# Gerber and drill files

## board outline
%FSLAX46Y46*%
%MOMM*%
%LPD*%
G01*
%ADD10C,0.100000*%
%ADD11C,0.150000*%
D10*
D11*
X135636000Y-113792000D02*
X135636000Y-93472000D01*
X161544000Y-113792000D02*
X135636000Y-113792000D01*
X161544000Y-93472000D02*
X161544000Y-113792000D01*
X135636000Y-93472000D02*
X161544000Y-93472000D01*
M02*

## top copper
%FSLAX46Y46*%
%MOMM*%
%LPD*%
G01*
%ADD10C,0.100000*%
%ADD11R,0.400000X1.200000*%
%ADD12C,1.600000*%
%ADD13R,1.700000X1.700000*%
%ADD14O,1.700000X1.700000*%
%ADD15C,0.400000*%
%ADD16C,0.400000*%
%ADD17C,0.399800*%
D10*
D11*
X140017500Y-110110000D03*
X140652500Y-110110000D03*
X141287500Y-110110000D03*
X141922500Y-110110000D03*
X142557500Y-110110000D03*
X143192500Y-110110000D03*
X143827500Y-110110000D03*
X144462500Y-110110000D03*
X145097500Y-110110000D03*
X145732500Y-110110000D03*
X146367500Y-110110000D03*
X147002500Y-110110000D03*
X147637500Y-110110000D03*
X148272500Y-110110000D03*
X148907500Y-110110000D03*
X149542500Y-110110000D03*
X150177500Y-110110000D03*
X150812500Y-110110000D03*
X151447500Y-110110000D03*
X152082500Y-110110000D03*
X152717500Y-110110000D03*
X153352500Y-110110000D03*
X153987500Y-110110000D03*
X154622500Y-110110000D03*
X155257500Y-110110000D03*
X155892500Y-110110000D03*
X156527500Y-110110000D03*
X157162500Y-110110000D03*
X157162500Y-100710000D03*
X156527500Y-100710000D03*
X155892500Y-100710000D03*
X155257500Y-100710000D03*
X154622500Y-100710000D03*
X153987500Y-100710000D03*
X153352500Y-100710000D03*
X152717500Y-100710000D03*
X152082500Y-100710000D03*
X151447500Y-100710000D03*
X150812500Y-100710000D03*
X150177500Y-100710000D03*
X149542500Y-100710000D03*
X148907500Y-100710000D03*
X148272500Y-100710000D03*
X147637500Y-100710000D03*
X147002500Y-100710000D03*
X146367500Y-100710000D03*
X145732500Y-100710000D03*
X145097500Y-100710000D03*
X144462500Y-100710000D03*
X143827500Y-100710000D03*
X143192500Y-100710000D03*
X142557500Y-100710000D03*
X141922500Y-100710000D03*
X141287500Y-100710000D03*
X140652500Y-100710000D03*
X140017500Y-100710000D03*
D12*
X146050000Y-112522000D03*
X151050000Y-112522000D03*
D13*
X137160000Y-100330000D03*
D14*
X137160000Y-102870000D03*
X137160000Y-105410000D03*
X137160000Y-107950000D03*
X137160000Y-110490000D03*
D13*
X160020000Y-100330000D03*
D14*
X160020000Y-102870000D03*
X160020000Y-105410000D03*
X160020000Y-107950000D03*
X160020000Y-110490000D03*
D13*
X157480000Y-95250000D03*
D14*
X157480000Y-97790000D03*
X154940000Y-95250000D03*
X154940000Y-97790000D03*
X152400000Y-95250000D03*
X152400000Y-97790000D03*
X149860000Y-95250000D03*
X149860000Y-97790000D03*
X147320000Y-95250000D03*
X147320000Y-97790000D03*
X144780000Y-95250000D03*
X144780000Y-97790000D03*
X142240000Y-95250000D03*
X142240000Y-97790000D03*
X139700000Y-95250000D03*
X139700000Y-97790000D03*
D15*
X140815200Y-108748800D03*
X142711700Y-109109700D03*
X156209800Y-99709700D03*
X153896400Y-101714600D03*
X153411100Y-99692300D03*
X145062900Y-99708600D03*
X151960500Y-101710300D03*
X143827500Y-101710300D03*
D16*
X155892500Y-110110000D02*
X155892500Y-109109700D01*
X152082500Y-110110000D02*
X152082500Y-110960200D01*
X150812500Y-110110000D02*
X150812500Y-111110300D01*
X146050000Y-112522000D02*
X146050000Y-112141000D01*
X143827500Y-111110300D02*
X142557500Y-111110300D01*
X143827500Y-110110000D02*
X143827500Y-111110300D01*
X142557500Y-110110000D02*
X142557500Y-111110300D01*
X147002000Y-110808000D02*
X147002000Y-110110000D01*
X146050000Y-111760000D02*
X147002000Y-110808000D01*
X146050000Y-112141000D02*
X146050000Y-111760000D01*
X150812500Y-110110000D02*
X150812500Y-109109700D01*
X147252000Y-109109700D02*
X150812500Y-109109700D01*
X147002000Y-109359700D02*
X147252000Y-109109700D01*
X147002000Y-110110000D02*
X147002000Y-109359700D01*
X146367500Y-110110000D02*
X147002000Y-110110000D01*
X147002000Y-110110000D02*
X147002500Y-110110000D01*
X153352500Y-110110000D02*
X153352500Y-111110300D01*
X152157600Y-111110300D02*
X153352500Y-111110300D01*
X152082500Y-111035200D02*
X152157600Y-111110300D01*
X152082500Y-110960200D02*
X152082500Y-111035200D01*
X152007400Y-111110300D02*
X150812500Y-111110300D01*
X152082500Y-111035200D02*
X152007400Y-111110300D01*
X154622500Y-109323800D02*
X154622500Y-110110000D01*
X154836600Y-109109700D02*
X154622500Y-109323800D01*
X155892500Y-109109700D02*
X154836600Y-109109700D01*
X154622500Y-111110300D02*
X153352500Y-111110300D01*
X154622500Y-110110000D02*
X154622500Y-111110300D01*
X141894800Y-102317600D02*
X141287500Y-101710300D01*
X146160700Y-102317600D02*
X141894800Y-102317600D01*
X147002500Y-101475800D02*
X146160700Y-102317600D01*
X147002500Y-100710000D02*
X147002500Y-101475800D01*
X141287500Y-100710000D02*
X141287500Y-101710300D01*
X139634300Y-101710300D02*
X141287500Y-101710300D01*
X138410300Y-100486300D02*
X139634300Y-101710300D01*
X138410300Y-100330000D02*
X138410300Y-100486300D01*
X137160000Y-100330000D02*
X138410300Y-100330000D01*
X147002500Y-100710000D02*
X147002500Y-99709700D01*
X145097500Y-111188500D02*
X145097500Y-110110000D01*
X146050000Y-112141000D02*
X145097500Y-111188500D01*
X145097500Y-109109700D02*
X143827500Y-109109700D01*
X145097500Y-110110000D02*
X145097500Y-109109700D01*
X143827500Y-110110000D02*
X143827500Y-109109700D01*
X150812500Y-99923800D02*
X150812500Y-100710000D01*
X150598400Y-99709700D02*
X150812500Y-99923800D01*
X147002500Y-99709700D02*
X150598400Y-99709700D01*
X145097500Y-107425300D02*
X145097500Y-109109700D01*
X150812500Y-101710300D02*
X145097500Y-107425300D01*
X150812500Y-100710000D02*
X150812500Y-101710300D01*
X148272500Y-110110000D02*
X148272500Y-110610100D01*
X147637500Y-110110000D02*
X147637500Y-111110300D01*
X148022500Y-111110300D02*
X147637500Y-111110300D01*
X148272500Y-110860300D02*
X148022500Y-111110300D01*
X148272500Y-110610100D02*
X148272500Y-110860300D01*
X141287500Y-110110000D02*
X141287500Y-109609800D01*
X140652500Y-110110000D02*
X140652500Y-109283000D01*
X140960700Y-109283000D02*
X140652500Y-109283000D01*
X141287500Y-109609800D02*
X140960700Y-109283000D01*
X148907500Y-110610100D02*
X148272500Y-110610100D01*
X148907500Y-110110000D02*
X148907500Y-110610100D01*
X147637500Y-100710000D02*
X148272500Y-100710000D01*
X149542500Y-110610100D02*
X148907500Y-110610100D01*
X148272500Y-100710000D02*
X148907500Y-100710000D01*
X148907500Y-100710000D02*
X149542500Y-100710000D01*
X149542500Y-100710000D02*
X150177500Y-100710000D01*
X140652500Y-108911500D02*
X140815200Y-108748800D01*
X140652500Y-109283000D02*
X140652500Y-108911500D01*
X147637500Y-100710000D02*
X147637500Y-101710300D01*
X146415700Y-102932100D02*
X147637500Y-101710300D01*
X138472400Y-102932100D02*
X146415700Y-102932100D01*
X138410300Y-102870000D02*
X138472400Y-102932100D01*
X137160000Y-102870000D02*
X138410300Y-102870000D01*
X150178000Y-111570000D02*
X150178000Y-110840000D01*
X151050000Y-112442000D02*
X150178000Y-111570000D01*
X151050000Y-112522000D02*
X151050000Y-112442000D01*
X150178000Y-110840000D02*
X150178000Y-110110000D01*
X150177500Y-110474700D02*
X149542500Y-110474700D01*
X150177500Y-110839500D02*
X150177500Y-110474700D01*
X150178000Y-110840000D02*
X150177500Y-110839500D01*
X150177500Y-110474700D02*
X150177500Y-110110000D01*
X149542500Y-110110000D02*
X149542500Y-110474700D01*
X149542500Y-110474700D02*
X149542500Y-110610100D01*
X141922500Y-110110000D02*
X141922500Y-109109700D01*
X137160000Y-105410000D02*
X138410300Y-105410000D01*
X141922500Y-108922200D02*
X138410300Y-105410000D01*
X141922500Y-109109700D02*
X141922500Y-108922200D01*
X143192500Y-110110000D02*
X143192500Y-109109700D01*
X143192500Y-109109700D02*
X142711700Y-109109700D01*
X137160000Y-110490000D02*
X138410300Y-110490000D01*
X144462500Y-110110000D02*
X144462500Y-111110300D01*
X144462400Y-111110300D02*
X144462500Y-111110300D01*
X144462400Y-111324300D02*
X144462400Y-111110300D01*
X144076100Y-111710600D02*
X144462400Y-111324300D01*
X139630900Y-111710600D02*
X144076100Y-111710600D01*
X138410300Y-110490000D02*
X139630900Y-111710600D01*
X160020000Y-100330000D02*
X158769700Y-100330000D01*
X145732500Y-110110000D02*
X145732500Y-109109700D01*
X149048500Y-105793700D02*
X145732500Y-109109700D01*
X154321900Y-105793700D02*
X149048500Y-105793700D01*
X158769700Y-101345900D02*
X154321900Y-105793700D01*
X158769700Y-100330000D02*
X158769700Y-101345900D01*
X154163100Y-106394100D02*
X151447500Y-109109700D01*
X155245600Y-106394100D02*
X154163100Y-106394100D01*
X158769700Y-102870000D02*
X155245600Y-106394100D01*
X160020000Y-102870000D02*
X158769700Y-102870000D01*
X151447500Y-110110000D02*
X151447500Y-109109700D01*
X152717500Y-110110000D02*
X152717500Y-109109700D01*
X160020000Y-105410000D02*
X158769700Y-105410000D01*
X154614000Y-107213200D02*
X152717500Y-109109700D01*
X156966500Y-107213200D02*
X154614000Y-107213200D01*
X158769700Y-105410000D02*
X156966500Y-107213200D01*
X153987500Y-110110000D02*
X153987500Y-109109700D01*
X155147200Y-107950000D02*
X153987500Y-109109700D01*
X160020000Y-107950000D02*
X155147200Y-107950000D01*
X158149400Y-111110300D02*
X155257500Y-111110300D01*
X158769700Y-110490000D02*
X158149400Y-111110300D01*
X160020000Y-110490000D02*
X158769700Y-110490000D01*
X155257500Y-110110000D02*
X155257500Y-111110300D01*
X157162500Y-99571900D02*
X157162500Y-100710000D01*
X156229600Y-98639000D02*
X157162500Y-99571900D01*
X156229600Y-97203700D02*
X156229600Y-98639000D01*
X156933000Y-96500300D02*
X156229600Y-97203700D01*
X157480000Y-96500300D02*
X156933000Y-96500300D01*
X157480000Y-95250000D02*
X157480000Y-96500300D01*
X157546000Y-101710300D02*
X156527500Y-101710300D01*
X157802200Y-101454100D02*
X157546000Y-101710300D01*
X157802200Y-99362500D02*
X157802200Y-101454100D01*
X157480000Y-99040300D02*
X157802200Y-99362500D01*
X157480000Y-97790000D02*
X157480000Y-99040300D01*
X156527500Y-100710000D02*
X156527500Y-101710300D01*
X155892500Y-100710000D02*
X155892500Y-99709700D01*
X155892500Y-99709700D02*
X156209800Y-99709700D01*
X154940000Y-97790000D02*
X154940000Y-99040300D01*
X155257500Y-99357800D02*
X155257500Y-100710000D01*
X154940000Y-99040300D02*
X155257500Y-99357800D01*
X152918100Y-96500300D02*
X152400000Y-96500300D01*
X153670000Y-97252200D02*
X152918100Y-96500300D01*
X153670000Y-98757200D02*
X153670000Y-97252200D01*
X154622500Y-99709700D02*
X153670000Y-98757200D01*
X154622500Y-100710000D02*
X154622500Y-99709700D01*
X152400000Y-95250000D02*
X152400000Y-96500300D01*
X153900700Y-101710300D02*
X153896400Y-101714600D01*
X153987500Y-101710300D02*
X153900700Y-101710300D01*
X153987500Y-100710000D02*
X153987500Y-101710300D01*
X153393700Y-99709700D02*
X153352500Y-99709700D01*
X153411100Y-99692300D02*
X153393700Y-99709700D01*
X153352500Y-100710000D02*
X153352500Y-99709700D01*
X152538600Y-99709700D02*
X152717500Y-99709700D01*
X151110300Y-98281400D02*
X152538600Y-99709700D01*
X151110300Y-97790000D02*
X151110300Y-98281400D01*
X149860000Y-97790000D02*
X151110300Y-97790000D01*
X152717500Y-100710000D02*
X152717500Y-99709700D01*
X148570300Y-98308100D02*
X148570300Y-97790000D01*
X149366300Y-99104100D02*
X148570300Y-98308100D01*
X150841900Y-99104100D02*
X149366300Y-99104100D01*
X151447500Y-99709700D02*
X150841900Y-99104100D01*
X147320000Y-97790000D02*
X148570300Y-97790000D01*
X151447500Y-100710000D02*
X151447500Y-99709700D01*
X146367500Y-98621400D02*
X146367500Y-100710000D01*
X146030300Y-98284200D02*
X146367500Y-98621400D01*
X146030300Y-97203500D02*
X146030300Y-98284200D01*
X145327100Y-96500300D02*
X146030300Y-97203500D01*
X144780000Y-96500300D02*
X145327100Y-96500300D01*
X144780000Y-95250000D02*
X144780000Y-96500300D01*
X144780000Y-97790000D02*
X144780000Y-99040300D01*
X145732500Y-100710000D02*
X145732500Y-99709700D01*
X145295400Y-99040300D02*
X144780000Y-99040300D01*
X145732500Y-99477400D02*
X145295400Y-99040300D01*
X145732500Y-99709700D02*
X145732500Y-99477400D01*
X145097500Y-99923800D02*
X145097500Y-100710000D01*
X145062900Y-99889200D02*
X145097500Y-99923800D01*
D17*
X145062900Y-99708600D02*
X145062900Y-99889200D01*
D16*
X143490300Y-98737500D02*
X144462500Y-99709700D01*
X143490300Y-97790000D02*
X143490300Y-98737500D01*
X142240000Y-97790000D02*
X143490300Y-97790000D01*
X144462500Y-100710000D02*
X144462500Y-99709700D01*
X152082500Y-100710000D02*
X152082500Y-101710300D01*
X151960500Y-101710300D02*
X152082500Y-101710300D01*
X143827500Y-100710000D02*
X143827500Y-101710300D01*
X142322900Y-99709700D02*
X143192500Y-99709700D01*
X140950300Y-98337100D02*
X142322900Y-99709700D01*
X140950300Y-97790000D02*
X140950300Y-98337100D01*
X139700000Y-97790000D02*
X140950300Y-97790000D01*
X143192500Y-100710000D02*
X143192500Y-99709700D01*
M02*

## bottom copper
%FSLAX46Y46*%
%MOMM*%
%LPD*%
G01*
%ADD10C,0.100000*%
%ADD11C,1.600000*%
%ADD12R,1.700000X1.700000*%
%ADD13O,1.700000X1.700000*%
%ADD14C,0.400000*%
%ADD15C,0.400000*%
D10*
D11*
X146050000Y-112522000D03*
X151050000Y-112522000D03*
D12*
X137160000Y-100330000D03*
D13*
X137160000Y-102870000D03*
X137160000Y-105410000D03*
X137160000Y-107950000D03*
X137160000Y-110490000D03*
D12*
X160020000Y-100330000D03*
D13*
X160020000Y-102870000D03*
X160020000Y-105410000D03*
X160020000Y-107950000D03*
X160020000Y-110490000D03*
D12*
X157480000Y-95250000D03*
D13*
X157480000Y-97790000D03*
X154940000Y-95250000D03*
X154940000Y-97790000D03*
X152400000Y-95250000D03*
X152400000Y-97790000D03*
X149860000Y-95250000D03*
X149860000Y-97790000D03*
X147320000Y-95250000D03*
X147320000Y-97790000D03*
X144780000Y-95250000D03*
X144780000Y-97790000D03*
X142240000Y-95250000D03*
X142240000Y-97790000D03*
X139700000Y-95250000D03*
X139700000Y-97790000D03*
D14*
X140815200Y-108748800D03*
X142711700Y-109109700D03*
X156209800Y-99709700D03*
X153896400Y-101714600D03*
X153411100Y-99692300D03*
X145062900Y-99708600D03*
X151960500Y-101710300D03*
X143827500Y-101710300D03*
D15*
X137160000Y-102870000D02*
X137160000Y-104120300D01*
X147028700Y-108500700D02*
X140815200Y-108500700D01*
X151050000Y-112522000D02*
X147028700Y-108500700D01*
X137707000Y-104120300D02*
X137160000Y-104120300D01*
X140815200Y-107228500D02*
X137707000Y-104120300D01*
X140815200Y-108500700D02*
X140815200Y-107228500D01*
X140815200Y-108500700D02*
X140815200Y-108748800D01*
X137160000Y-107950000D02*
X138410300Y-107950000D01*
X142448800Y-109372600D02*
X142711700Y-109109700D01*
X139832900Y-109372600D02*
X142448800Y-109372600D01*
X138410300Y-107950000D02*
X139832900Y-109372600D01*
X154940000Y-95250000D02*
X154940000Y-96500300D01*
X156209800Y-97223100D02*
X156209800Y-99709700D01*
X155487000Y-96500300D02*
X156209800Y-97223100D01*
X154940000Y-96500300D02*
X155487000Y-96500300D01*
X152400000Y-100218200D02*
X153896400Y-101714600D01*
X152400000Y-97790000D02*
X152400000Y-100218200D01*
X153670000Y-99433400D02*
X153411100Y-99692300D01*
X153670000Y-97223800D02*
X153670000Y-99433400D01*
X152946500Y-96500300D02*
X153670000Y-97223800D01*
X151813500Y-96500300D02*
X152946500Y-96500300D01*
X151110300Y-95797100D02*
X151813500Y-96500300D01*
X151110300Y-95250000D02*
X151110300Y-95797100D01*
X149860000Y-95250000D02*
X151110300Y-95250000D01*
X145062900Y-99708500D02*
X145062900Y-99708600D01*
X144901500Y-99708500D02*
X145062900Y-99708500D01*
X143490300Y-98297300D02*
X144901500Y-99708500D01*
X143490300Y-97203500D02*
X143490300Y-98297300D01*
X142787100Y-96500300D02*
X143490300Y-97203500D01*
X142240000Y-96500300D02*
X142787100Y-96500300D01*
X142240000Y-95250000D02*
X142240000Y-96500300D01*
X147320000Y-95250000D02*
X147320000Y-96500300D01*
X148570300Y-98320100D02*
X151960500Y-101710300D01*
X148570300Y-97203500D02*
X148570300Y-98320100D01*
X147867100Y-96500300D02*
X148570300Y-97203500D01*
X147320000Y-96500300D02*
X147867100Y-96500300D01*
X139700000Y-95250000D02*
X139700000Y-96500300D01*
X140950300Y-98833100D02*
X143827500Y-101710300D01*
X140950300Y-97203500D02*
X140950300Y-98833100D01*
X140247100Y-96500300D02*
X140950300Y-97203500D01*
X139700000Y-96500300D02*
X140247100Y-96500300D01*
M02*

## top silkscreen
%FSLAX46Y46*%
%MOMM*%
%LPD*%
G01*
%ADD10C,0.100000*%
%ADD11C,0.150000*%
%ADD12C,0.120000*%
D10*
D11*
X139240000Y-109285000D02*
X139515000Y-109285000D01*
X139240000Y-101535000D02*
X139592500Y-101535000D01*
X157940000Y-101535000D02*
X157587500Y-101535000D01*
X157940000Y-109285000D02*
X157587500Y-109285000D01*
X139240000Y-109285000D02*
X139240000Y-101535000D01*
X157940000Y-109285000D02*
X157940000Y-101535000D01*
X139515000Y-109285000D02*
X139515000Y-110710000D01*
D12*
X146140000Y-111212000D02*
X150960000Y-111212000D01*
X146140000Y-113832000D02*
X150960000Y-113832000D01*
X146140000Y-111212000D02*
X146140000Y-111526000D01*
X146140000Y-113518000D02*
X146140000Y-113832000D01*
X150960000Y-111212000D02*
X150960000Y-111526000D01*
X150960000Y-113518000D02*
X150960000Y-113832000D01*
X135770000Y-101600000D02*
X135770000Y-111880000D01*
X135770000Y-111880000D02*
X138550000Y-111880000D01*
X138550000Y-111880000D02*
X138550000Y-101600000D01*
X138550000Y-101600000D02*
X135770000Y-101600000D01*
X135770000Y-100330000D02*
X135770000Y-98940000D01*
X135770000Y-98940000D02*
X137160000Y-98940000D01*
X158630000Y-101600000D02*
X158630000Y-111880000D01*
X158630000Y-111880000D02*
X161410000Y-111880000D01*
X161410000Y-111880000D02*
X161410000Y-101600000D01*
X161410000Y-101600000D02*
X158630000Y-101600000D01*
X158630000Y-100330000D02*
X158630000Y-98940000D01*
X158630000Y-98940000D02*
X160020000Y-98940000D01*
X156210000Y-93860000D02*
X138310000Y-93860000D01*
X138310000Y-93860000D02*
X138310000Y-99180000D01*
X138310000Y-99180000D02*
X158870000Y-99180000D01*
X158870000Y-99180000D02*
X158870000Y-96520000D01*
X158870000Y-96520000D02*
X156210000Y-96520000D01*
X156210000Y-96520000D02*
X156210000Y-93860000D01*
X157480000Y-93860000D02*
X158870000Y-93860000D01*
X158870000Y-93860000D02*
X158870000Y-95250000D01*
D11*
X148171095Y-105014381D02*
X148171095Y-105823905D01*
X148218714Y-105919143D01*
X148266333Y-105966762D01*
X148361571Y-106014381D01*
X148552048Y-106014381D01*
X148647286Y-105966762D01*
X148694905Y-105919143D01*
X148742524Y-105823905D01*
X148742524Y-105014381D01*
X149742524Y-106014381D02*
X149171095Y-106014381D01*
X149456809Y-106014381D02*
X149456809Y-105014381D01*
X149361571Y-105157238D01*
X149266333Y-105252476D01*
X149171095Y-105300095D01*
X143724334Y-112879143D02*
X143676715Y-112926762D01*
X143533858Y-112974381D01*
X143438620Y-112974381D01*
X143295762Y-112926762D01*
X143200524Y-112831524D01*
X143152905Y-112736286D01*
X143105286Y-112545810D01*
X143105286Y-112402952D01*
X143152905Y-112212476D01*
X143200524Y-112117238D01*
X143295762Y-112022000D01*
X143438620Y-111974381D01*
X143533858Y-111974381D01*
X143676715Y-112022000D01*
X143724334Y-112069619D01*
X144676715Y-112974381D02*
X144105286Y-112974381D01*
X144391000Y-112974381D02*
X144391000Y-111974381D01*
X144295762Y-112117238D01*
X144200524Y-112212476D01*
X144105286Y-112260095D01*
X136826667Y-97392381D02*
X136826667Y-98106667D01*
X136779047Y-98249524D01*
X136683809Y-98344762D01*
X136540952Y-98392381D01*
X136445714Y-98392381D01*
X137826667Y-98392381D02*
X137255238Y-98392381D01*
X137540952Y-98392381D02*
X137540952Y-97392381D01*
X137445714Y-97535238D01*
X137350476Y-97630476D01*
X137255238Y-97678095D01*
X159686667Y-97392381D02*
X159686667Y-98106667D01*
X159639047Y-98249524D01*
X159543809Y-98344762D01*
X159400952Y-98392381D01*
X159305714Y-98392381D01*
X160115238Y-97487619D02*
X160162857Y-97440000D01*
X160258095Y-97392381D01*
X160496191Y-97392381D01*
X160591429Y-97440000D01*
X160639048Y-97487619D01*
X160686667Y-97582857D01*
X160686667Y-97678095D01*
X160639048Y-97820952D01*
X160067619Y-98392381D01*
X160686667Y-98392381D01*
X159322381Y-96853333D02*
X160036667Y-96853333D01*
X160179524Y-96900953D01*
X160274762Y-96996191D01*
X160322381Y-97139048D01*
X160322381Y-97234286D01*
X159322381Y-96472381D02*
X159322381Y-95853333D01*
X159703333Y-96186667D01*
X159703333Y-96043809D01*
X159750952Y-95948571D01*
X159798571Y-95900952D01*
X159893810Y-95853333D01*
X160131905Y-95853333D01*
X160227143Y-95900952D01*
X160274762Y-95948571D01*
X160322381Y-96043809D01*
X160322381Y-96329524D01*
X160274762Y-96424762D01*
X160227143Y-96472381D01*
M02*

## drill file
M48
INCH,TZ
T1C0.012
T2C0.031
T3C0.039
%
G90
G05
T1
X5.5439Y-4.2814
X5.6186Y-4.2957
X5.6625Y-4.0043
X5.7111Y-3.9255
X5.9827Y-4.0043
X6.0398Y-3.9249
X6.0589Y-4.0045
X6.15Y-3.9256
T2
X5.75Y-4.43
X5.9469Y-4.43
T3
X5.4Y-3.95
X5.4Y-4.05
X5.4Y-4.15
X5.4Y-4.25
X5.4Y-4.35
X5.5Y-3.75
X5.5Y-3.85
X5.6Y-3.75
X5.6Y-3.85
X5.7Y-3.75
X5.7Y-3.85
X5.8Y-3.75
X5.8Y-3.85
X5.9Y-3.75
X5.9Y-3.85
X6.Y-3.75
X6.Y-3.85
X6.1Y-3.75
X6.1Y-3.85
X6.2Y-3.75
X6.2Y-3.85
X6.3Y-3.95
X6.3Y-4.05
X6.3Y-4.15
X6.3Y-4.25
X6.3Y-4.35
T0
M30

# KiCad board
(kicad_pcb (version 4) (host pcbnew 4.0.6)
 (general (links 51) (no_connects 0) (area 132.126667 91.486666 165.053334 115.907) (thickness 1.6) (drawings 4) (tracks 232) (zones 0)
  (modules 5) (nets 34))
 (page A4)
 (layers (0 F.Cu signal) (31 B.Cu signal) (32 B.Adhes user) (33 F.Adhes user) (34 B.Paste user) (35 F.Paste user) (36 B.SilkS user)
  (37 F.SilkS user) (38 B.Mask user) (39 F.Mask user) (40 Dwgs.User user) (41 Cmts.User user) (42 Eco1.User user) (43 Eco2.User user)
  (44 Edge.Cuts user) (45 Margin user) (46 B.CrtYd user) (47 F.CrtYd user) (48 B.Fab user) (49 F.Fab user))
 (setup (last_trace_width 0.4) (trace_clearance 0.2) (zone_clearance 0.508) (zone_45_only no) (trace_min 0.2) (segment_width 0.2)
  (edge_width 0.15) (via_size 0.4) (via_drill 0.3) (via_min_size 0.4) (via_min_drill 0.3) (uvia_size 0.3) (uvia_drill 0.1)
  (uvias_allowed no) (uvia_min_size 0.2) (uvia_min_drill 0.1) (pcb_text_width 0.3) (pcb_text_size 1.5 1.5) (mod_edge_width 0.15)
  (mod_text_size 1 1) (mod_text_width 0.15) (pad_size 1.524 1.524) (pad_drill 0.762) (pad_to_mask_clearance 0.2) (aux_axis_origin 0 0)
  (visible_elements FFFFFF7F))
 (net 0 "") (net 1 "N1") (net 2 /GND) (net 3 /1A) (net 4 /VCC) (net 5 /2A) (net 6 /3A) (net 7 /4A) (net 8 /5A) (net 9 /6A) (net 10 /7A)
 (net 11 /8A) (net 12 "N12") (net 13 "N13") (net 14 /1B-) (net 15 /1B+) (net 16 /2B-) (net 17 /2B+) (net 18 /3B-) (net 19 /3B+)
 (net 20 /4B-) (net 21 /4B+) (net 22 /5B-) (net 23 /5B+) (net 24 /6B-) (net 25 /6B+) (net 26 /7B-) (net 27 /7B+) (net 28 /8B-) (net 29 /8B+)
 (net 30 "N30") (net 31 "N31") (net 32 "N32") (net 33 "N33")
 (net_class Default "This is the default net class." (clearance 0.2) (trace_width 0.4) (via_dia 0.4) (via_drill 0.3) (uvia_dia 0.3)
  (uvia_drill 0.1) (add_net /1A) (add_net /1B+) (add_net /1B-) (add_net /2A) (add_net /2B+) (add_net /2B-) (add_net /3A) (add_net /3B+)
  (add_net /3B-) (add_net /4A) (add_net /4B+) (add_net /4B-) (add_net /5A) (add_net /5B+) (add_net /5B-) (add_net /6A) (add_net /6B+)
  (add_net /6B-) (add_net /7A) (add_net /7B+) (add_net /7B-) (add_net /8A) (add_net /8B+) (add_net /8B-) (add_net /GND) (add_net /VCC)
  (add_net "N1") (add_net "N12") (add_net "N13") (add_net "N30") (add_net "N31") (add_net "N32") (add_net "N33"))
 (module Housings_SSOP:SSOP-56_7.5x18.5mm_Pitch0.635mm (layer F.Cu) (at 148.59 105.41 90)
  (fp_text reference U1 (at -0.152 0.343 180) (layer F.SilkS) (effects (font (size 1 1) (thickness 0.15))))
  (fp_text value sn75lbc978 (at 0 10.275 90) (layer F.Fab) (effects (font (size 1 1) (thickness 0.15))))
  (fp_line (start -3.875 -9.35) (end -3.875 -9.075) (layer F.SilkS) (width 0.15))
  (fp_line (start 3.875 -9.35) (end 3.875 -8.9975) (layer F.SilkS) (width 0.15))
  (fp_line (start 3.875 9.35) (end 3.875 8.9975) (layer F.SilkS) (width 0.15))
  (fp_line (start -3.875 9.35) (end -3.875 8.9975) (layer F.SilkS) (width 0.15))
  (fp_line (start -3.875 -9.35) (end 3.875 -9.35) (layer F.SilkS) (width 0.15))
  (fp_line (start -3.875 9.35) (end 3.875 9.35) (layer F.SilkS) (width 0.15))
  (fp_line (start -3.875 -9.075) (end -5.3 -9.075) (layer F.SilkS) (width 0.15))
  (pad 1 smd rect (at -4.7 -8.5725 90) (size 1.2 0.4) (layers F.Cu F.Paste F.Mask) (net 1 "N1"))
  (pad 2 smd rect (at -4.7 -7.9375 90) (size 1.2 0.4) (layers F.Cu F.Paste F.Mask) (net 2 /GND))
  (pad 3 smd rect (at -4.7 -7.3025 90) (size 1.2 0.4) (layers F.Cu F.Paste F.Mask) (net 2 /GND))
  (pad 4 smd rect (at -4.7 -6.6675 90) (size 1.2 0.4) (layers F.Cu F.Paste F.Mask) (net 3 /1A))
  (pad 5 smd rect (at -4.7 -6.0325 90) (size 1.2 0.4) (layers F.Cu F.Paste F.Mask) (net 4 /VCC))
  (pad 6 smd rect (at -4.7 -5.3975 90) (size 1.2 0.4) (layers F.Cu F.Paste F.Mask) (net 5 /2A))
  (pad 7 smd rect (at -4.7 -4.7625 90) (size 1.2 0.4) (layers F.Cu F.Paste F.Mask) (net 4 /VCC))
  (pad 8 smd rect (at -4.7 -4.1275 90) (size 1.2 0.4) (layers F.Cu F.Paste F.Mask) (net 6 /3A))
  (pad 9 smd rect (at -4.7 -3.4925 90) (size 1.2 0.4) (layers F.Cu F.Paste F.Mask) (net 4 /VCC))
  (pad 10 smd rect (at -4.7 -2.8575 90) (size 1.2 0.4) (layers F.Cu F.Paste F.Mask) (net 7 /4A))
  (pad 11 smd rect (at -4.7 -2.2225 90) (size 1.2 0.4) (layers F.Cu F.Paste F.Mask) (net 4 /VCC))
  (pad 12 smd rect (at -4.7 -1.5875 90) (size 1.2 0.4) (layers F.Cu F.Paste F.Mask) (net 4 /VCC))
  (pad 13 smd rect (at -4.7 -0.9525 90) (size 1.2 0.4) (layers F.Cu F.Paste F.Mask) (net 2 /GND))
  (pad 14 smd rect (at -4.7 -0.3175 90) (size 1.2 0.4) (layers F.Cu F.Paste F.Mask) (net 2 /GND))
  (pad 15 smd rect (at -4.7 0.3175 90) (size 1.2 0.4) (layers F.Cu F.Paste F.Mask) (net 2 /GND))
  (pad 16 smd rect (at -4.7 0.9525 90) (size 1.2 0.4) (layers F.Cu F.Paste F.Mask) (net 2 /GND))
  (pad 17 smd rect (at -4.7 1.5875 90) (size 1.2 0.4) (layers F.Cu F.Paste F.Mask) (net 2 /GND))
  (pad 18 smd rect (at -4.7 2.2225 90) (size 1.2 0.4) (layers F.Cu F.Paste F.Mask) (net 4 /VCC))
  (pad 19 smd rect (at -4.7 2.8575 90) (size 1.2 0.4) (layers F.Cu F.Paste F.Mask) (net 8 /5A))
  (pad 20 smd rect (at -4.7 3.4925 90) (size 1.2 0.4) (layers F.Cu F.Paste F.Mask) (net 4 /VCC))
  (pad 21 smd rect (at -4.7 4.1275 90) (size 1.2 0.4) (layers F.Cu F.Paste F.Mask) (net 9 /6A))
  (pad 22 smd rect (at -4.7 4.7625 90) (size 1.2 0.4) (layers F.Cu F.Paste F.Mask) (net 4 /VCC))
  (pad 23 smd rect (at -4.7 5.3975 90) (size 1.2 0.4) (layers F.Cu F.Paste F.Mask) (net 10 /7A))
  (pad 24 smd rect (at -4.7 6.0325 90) (size 1.2 0.4) (layers F.Cu F.Paste F.Mask) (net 4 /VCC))
  (pad 25 smd rect (at -4.7 6.6675 90) (size 1.2 0.4) (layers F.Cu F.Paste F.Mask) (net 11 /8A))
  (pad 26 smd rect (at -4.7 7.3025 90) (size 1.2 0.4) (layers F.Cu F.Paste F.Mask) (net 4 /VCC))
  (pad 27 smd rect (at -4.7 7.9375 90) (size 1.2 0.4) (layers F.Cu F.Paste F.Mask) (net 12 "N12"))
  (pad 28 smd rect (at -4.7 8.5725 90) (size 1.2 0.4) (layers F.Cu F.Paste F.Mask) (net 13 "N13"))
  (pad 29 smd rect (at 4.7 8.5725 90) (size 1.2 0.4) (layers F.Cu F.Paste F.Mask) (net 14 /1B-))
  (pad 30 smd rect (at 4.7 7.9375 90) (size 1.2 0.4) (layers F.Cu F.Paste F.Mask) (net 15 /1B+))
  (pad 31 smd rect (at 4.7 7.3025 90) (size 1.2 0.4) (layers F.Cu F.Paste F.Mask) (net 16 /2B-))
  (pad 32 smd rect (at 4.7 6.6675 90) (size 1.2 0.4) (layers F.Cu F.Paste F.Mask) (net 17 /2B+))
  (pad 33 smd rect (at 4.7 6.0325 90) (size 1.2 0.4) (layers F.Cu F.Paste F.Mask) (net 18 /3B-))
  (pad 34 smd rect (at 4.7 5.3975 90) (size 1.2 0.4) (layers F.Cu F.Paste F.Mask) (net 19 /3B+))
  (pad 35 smd rect (at 4.7 4.7625 90) (size 1.2 0.4) (layers F.Cu F.Paste F.Mask) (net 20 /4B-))
  (pad 36 smd rect (at 4.7 4.1275 90) (size 1.2 0.4) (layers F.Cu F.Paste F.Mask) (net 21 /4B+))
  (pad 37 smd rect (at 4.7 3.4925 90) (size 1.2 0.4) (layers F.Cu F.Paste F.Mask) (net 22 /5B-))
  (pad 38 smd rect (at 4.7 2.8575 90) (size 1.2 0.4) (layers F.Cu F.Paste F.Mask) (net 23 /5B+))
  (pad 39 smd rect (at 4.7 2.2225 90) (size 1.2 0.4) (layers F.Cu F.Paste F.Mask) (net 4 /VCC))
  (pad 40 smd rect (at 4.7 1.5875 90) (size 1.2 0.4) (layers F.Cu F.Paste F.Mask) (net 2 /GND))
  (pad 41 smd rect (at 4.7 0.9525 90) (size 1.2 0.4) (layers F.Cu F.Paste F.Mask) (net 2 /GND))
  (pad 42 smd rect (at 4.7 0.3175 90) (size 1.2 0.4) (layers F.Cu F.Paste F.Mask) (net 2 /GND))
  (pad 43 smd rect (at 4.7 -0.3175 90) (size 1.2 0.4) (layers F.Cu F.Paste F.Mask) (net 2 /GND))
  (pad 44 smd rect (at 4.7 -0.9525 90) (size 1.2 0.4) (layers F.Cu F.Paste F.Mask) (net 2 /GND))
  (pad 45 smd rect (at 4.7 -1.5875 90) (size 1.2 0.4) (layers F.Cu F.Paste F.Mask) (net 4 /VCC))
  (pad 46 smd rect (at 4.7 -2.2225 90) (size 1.2 0.4) (layers F.Cu F.Paste F.Mask) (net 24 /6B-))
  (pad 47 smd rect (at 4.7 -2.8575 90) (size 1.2 0.4) (layers F.Cu F.Paste F.Mask) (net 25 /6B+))
  (pad 48 smd rect (at 4.7 -3.4925 90) (size 1.2 0.4) (layers F.Cu F.Paste F.Mask) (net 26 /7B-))
  (pad 49 smd rect (at 4.7 -4.1275 90) (size 1.2 0.4) (layers F.Cu F.Paste F.Mask) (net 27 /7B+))
  (pad 50 smd rect (at 4.7 -4.7625 90) (size 1.2 0.4) (layers F.Cu F.Paste F.Mask) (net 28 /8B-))
  (pad 51 smd rect (at 4.7 -5.3975 90) (size 1.2 0.4) (layers F.Cu F.Paste F.Mask) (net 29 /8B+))
  (pad 52 smd rect (at 4.7 -6.0325 90) (size 1.2 0.4) (layers F.Cu F.Paste F.Mask) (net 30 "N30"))
  (pad 53 smd rect (at 4.7 -6.6675 90) (size 1.2 0.4) (layers F.Cu F.Paste F.Mask) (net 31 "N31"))
  (pad 54 smd rect (at 4.7 -7.3025 90) (size 1.2 0.4) (layers F.Cu F.Paste F.Mask) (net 4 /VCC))
  (pad 55 smd rect (at 4.7 -7.9375 90) (size 1.2 0.4) (layers F.Cu F.Paste F.Mask) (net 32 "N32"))
  (pad 56 smd rect (at 4.7 -8.5725 90) (size 1.2 0.4) (layers F.Cu F.Paste F.Mask) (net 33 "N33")))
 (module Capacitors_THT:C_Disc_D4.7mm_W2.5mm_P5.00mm (layer F.Cu) (at 146.05 112.522)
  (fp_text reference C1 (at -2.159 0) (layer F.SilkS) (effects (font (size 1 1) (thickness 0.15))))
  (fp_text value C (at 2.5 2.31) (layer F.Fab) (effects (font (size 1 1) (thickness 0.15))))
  (fp_line (start 0.09 -1.31) (end 4.91 -1.31) (layer F.SilkS) (width 0.12))
  (fp_line (start 0.09 1.31) (end 4.91 1.31) (layer F.SilkS) (width 0.12))
  (fp_line (start 0.09 -1.31) (end 0.09 -0.996) (layer F.SilkS) (width 0.12))
  (fp_line (start 0.09 0.996) (end 0.09 1.31) (layer F.SilkS) (width 0.12))
  (fp_line (start 4.91 -1.31) (end 4.91 -0.996) (layer F.SilkS) (width 0.12))
  (fp_line (start 4.91 0.996) (end 4.91 1.31) (layer F.SilkS) (width 0.12))
  (pad 1 thru_hole circle (at 0 0) (size 1.6 1.6) (drill 0.8) (layers *.Cu *.Mask) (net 4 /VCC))
  (pad 2 thru_hole circle (at 5 0) (size 1.6 1.6) (drill 0.8) (layers *.Cu *.Mask) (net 2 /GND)))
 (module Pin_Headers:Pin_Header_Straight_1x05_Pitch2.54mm (layer F.Cu) (at 137.16 100.33)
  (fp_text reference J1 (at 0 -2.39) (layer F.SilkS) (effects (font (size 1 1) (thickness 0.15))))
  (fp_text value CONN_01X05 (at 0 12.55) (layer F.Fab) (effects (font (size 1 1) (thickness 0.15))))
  (fp_line (start -1.39 1.27) (end -1.39 11.55) (layer F.SilkS) (width 0.12))
  (fp_line (start -1.39 11.55) (end 1.39 11.55) (layer F.SilkS) (width 0.12))
  (fp_line (start 1.39 11.55) (end 1.39 1.27) (layer F.SilkS) (width 0.12))
  (fp_line (start 1.39 1.27) (end -1.39 1.27) (layer F.SilkS) (width 0.12))
  (fp_line (start -1.39 0) (end -1.39 -1.39) (layer F.SilkS) (width 0.12))
  (fp_line (start -1.39 -1.39) (end 0 -1.39) (layer F.SilkS) (width 0.12))
  (pad 1 thru_hole rect (at 0 0) (size 1.7 1.7) (drill 1) (layers *.Cu *.Mask) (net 4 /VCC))
  (pad 2 thru_hole oval (at 0 2.54) (size 1.7 1.7) (drill 1) (layers *.Cu *.Mask) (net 2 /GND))
  (pad 3 thru_hole oval (at 0 5.08) (size 1.7 1.7) (drill 1) (layers *.Cu *.Mask) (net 3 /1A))
  (pad 4 thru_hole oval (at 0 7.62) (size 1.7 1.7) (drill 1) (layers *.Cu *.Mask) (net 5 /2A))
  (pad 5 thru_hole oval (at 0 10.16) (size 1.7 1.7) (drill 1) (layers *.Cu *.Mask) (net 6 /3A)))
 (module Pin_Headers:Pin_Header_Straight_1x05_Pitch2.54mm (layer F.Cu) (at 160.02 100.33)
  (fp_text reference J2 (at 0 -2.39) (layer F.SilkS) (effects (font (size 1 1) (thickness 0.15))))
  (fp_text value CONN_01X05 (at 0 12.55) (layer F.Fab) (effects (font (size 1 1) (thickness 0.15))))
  (fp_line (start -1.39 1.27) (end -1.39 11.55) (layer F.SilkS) (width 0.12))
  (fp_line (start -1.39 11.55) (end 1.39 11.55) (layer F.SilkS) (width 0.12))
  (fp_line (start 1.39 11.55) (end 1.39 1.27) (layer F.SilkS) (width 0.12))
  (fp_line (start 1.39 1.27) (end -1.39 1.27) (layer F.SilkS) (width 0.12))
  (fp_line (start -1.39 0) (end -1.39 -1.39) (layer F.SilkS) (width 0.12))
  (fp_line (start -1.39 -1.39) (end 0 -1.39) (layer F.SilkS) (width 0.12))
  (pad 1 thru_hole rect (at 0 0) (size 1.7 1.7) (drill 1) (layers *.Cu *.Mask) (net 7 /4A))
  (pad 2 thru_hole oval (at 0 2.54) (size 1.7 1.7) (drill 1) (layers *.Cu *.Mask) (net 8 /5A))
  (pad 3 thru_hole oval (at 0 5.08) (size 1.7 1.7) (drill 1) (layers *.Cu *.Mask) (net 9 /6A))
  (pad 4 thru_hole oval (at 0 7.62) (size 1.7 1.7) (drill 1) (layers *.Cu *.Mask) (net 10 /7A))
  (pad 5 thru_hole oval (at 0 10.16) (size 1.7 1.7) (drill 1) (layers *.Cu *.Mask) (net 11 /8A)))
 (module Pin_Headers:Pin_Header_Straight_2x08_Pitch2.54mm (layer F.Cu) (at 157.48 95.25 270)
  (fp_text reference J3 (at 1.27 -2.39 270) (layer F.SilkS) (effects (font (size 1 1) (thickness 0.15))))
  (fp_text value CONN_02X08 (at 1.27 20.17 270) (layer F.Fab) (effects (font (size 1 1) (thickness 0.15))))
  (fp_line (start -1.39 1.27) (end -1.39 19.17) (layer F.SilkS) (width 0.12))
  (fp_line (start -1.39 19.17) (end 3.93 19.17) (layer F.SilkS) (width 0.12))
  (fp_line (start 3.93 19.17) (end 3.93 -1.39) (layer F.SilkS) (width 0.12))
  (fp_line (start 3.93 -1.39) (end 1.27 -1.39) (layer F.SilkS) (width 0.12))
  (fp_line (start 1.27 -1.39) (end 1.27 1.27) (layer F.SilkS) (width 0.12))
  (fp_line (start 1.27 1.27) (end -1.39 1.27) (layer F.SilkS) (width 0.12))
  (fp_line (start -1.39 0) (end -1.39 -1.39) (layer F.SilkS) (width 0.12))
  (fp_line (start -1.39 -1.39) (end 0 -1.39) (layer F.SilkS) (width 0.12))
  (pad 1 thru_hole rect (at 0 0 270) (size 1.7 1.7) (drill 1) (layers *.Cu *.Mask) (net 14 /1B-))
  (pad 2 thru_hole oval (at 2.54 0 270) (size 1.7 1.7) (drill 1) (layers *.Cu *.Mask) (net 15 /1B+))
  (pad 3 thru_hole oval (at 0 2.54 270) (size 1.7 1.7) (drill 1) (layers *.Cu *.Mask) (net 16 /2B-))
  (pad 4 thru_hole oval (at 2.54 2.54 270) (size 1.7 1.7) (drill 1) (layers *.Cu *.Mask) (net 17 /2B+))
  (pad 5 thru_hole oval (at 0 5.08 270) (size 1.7 1.7) (drill 1) (layers *.Cu *.Mask) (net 18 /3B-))
  (pad 6 thru_hole oval (at 2.54 5.08 270) (size 1.7 1.7) (drill 1) (layers *.Cu *.Mask) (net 19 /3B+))
  (pad 7 thru_hole oval (at 0 7.62 270) (size 1.7 1.7) (drill 1) (layers *.Cu *.Mask) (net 20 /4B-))
  (pad 8 thru_hole oval (at 2.54 7.62 270) (size 1.7 1.7) (drill 1) (layers *.Cu *.Mask) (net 21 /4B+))
  (pad 9 thru_hole oval (at 0 10.16 270) (size 1.7 1.7) (drill 1) (layers *.Cu *.Mask) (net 22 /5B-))
  (pad 10 thru_hole oval (at 2.54 10.16 270) (size 1.7 1.7) (drill 1) (layers *.Cu *.Mask) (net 23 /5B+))
  (pad 11 thru_hole oval (at 0 12.7 270) (size 1.7 1.7) (drill 1) (layers *.Cu *.Mask) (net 24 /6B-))
  (pad 12 thru_hole oval (at 2.54 12.7 270) (size 1.7 1.7) (drill 1) (layers *.Cu *.Mask) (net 25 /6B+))
  (pad 13 thru_hole oval (at 0 15.24 270) (size 1.7 1.7) (drill 1) (layers *.Cu *.Mask) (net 26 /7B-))
  (pad 14 thru_hole oval (at 2.54 15.24 270) (size 1.7 1.7) (drill 1) (layers *.Cu *.Mask) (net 27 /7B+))
  (pad 15 thru_hole oval (at 0 17.78 270) (size 1.7 1.7) (drill 1) (layers *.Cu *.Mask) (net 28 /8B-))
  (pad 16 thru_hole oval (at 2.54 17.78 270) (size 1.7 1.7) (drill 1) (layers *.Cu *.Mask) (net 29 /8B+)))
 (gr_line (start 135.636 113.792) (end 135.636 93.472) (angle 90) (layer Edge.Cuts) (width 0.15))
 (gr_line (start 161.544 113.792) (end 135.636 113.792) (angle 90) (layer Edge.Cuts) (width 0.15))
 (gr_line (start 161.544 93.472) (end 161.544 113.792) (angle 90) (layer Edge.Cuts) (width 0.15))
 (gr_line (start 135.636 93.472) (end 161.544 93.472) (angle 90) (layer Edge.Cuts) (width 0.15))
 (segment (start 155.8925 110.11) (end 155.8925 109.1097) (width 0.4) (layer F.Cu) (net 4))
 (segment (start 152.0825 110.11) (end 152.0825 110.9602) (width 0.4) (layer F.Cu) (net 4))
 (segment (start 150.8125 110.11) (end 150.8125 111.1103) (width 0.4) (layer F.Cu) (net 4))
 (segment (start 146.05 112.522) (end 146.05 112.141) (width 0.4) (layer F.Cu) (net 4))
 (segment (start 143.8275 111.1103) (end 142.5575 111.1103) (width 0.4) (layer F.Cu) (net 4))
 (segment (start 143.8275 110.11) (end 143.8275 111.1103) (width 0.4) (layer F.Cu) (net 4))
 (segment (start 142.5575 110.11) (end 142.5575 111.1103) (width 0.4) (layer F.Cu) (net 4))
 (segment (start 147.002 110.808) (end 147.002 110.11) (width 0.4) (layer F.Cu) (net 4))
 (segment (start 146.05 111.76) (end 147.002 110.808) (width 0.4) (layer F.Cu) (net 4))
 (segment (start 146.05 112.141) (end 146.05 111.76) (width 0.4) (layer F.Cu) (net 4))
 (segment (start 150.8125 110.11) (end 150.8125 109.1097) (width 0.4) (layer F.Cu) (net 4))
 (segment (start 147.252 109.1097) (end 150.8125 109.1097) (width 0.4) (layer F.Cu) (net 4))
 (segment (start 147.002 109.3597) (end 147.252 109.1097) (width 0.4) (layer F.Cu) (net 4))
 (segment (start 147.002 110.11) (end 147.002 109.3597) (width 0.4) (layer F.Cu) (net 4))
 (segment (start 146.3675 110.11) (end 147.002 110.11) (width 0.4) (layer F.Cu) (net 4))
 (segment (start 147.002 110.11) (end 147.0025 110.11) (width 0.4) (layer F.Cu) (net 4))
 (segment (start 153.3525 110.11) (end 153.3525 111.1103) (width 0.4) (layer F.Cu) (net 4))
 (segment (start 152.1576 111.1103) (end 153.3525 111.1103) (width 0.4) (layer F.Cu) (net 4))
 (segment (start 152.0825 111.0352) (end 152.1576 111.1103) (width 0.4) (layer F.Cu) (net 4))
 (segment (start 152.0825 110.9602) (end 152.0825 111.0352) (width 0.4) (layer F.Cu) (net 4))
 (segment (start 152.0074 111.1103) (end 150.8125 111.1103) (width 0.4) (layer F.Cu) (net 4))
 (segment (start 152.0825 111.0352) (end 152.0074 111.1103) (width 0.4) (layer F.Cu) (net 4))
 (segment (start 154.6225 109.3238) (end 154.6225 110.11) (width 0.4) (layer F.Cu) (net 4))
 (segment (start 154.8366 109.1097) (end 154.6225 109.3238) (width 0.4) (layer F.Cu) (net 4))
 (segment (start 155.8925 109.1097) (end 154.8366 109.1097) (width 0.4) (layer F.Cu) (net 4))
 (segment (start 154.6225 111.1103) (end 153.3525 111.1103) (width 0.4) (layer F.Cu) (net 4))
 (segment (start 154.6225 110.11) (end 154.6225 111.1103) (width 0.4) (layer F.Cu) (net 4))
 (segment (start 141.8948 102.3176) (end 141.2875 101.7103) (width 0.4) (layer F.Cu) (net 4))
 (segment (start 146.1607 102.3176) (end 141.8948 102.3176) (width 0.4) (layer F.Cu) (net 4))
 (segment (start 147.0025 101.4758) (end 146.1607 102.3176) (width 0.4) (layer F.Cu) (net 4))
 (segment (start 147.0025 100.71) (end 147.0025 101.4758) (width 0.4) (layer F.Cu) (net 4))
 (segment (start 141.2875 100.71) (end 141.2875 101.7103) (width 0.4) (layer F.Cu) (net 4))
 (segment (start 139.6343 101.7103) (end 141.2875 101.7103) (width 0.4) (layer F.Cu) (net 4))
 (segment (start 138.4103 100.4863) (end 139.6343 101.7103) (width 0.4) (layer F.Cu) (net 4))
 (segment (start 138.4103 100.33) (end 138.4103 100.4863) (width 0.4) (layer F.Cu) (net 4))
 (segment (start 137.16 100.33) (end 138.4103 100.33) (width 0.4) (layer F.Cu) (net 4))
 (segment (start 147.0025 100.71) (end 147.0025 99.7097) (width 0.4) (layer F.Cu) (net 4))
 (segment (start 145.0975 111.1885) (end 145.0975 110.11) (width 0.4) (layer F.Cu) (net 4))
 (segment (start 146.05 112.141) (end 145.0975 111.1885) (width 0.4) (layer F.Cu) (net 4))
 (segment (start 145.0975 109.1097) (end 143.8275 109.1097) (width 0.4) (layer F.Cu) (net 4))
 (segment (start 145.0975 110.11) (end 145.0975 109.1097) (width 0.4) (layer F.Cu) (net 4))
 (segment (start 143.8275 110.11) (end 143.8275 109.1097) (width 0.4) (layer F.Cu) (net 4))
 (segment (start 150.8125 99.9238) (end 150.8125 100.71) (width 0.4) (layer F.Cu) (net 4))
 (segment (start 150.5984 99.7097) (end 150.8125 99.9238) (width 0.4) (layer F.Cu) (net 4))
 (segment (start 147.0025 99.7097) (end 150.5984 99.7097) (width 0.4) (layer F.Cu) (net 4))
 (segment (start 145.0975 107.4253) (end 145.0975 109.1097) (width 0.4) (layer F.Cu) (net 4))
 (segment (start 150.8125 101.7103) (end 145.0975 107.4253) (width 0.4) (layer F.Cu) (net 4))
 (segment (start 150.8125 100.71) (end 150.8125 101.7103) (width 0.4) (layer F.Cu) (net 4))
 (via (at 140.8152 108.7488) (size 0.4) (layers F.Cu B.Cu) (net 2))
 (segment (start 148.2725 110.11) (end 148.2725 110.6101) (width 0.4) (layer F.Cu) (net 2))
 (segment (start 147.6375 110.11) (end 147.6375 111.1103) (width 0.4) (layer F.Cu) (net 2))
 (segment (start 148.0225 111.1103) (end 147.6375 111.1103) (width 0.4) (layer F.Cu) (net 2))
 (segment (start 148.2725 110.8603) (end 148.0225 111.1103) (width 0.4) (layer F.Cu) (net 2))
 (segment (start 148.2725 110.6101) (end 148.2725 110.8603) (width 0.4) (layer F.Cu) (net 2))
 (segment (start 141.2875 110.11) (end 141.2875 109.6098) (width 0.4) (layer F.Cu) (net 2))
 (segment (start 140.6525 110.11) (end 140.6525 109.283) (width 0.4) (layer F.Cu) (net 2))
 (segment (start 140.9607 109.283) (end 140.6525 109.283) (width 0.4) (layer F.Cu) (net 2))
 (segment (start 141.2875 109.6098) (end 140.9607 109.283) (width 0.4) (layer F.Cu) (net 2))
 (segment (start 137.16 102.87) (end 137.16 104.1203) (width 0.4) (layer B.Cu) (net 2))
 (segment (start 148.9075 110.6101) (end 148.2725 110.6101) (width 0.4) (layer F.Cu) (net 2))
 (segment (start 148.9075 110.11) (end 148.9075 110.6101) (width 0.4) (layer F.Cu) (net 2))
 (segment (start 147.6375 100.71) (end 148.2725 100.71) (width 0.4) (layer F.Cu) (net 2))
 (segment (start 149.5425 110.6101) (end 148.9075 110.6101) (width 0.4) (layer F.Cu) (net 2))
 (segment (start 148.2725 100.71) (end 148.9075 100.71) (width 0.4) (layer F.Cu) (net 2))
 (segment (start 148.9075 100.71) (end 149.5425 100.71) (width 0.4) (layer F.Cu) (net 2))
 (segment (start 149.5425 100.71) (end 150.1775 100.71) (width 0.4) (layer F.Cu) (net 2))
 (segment (start 147.0287 108.5007) (end 140.8152 108.5007) (width 0.4) (layer B.Cu) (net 2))
 (segment (start 151.05 112.522) (end 147.0287 108.5007) (width 0.4) (layer B.Cu) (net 2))
 (segment (start 137.707 104.1203) (end 137.16 104.1203) (width 0.4) (layer B.Cu) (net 2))
 (segment (start 140.8152 107.2285) (end 137.707 104.1203) (width 0.4) (layer B.Cu) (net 2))
 (segment (start 140.8152 108.5007) (end 140.8152 107.2285) (width 0.4) (layer B.Cu) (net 2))
 (segment (start 140.8152 108.5007) (end 140.8152 108.7488) (width 0.4) (layer B.Cu) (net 2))
 (segment (start 140.6525 108.9115) (end 140.8152 108.7488) (width 0.4) (layer F.Cu) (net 2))
 (segment (start 140.6525 109.283) (end 140.6525 108.9115) (width 0.4) (layer F.Cu) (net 2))
 (segment (start 147.6375 100.71) (end 147.6375 101.7103) (width 0.4) (layer F.Cu) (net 2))
 (segment (start 146.4157 102.9321) (end 147.6375 101.7103) (width 0.4) (layer F.Cu) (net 2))
 (segment (start 138.4724 102.9321) (end 146.4157 102.9321) (width 0.4) (layer F.Cu) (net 2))
 (segment (start 138.4103 102.87) (end 138.4724 102.9321) (width 0.4) (layer F.Cu) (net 2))
 (segment (start 137.16 102.87) (end 138.4103 102.87) (width 0.4) (layer F.Cu) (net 2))
 (segment (start 150.178 111.57) (end 150.178 110.84) (width 0.4) (layer F.Cu) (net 2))
 (segment (start 151.05 112.442) (end 150.178 111.57) (width 0.4) (layer F.Cu) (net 2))
 (segment (start 151.05 112.522) (end 151.05 112.442) (width 0.4) (layer F.Cu) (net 2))
 (segment (start 150.178 110.84) (end 150.178 110.11) (width 0.4) (layer F.Cu) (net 2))
 (segment (start 150.1775 110.4747) (end 149.5425 110.4747) (width 0.4) (layer F.Cu) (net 2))
 (segment (start 150.1775 110.8395) (end 150.1775 110.4747) (width 0.4) (layer F.Cu) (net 2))
 (segment (start 150.178 110.84) (end 150.1775 110.8395) (width 0.4) (layer F.Cu) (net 2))
 (segment (start 150.1775 110.4747) (end 150.1775 110.11) (width 0.4) (layer F.Cu) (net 2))
 (segment (start 149.5425 110.11) (end 149.5425 110.4747) (width 0.4) (layer F.Cu) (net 2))
 (segment (start 149.5425 110.4747) (end 149.5425 110.6101) (width 0.4) (layer F.Cu) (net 2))
 (segment (start 141.9225 110.11) (end 141.9225 109.1097) (width 0.4) (layer F.Cu) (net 3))
 (segment (start 137.16 105.41) (end 138.4103 105.41) (width 0.4) (layer F.Cu) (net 3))
 (segment (start 141.9225 108.9222) (end 138.4103 105.41) (width 0.4) (layer F.Cu) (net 3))
 (segment (start 141.9225 109.1097) (end 141.9225 108.9222) (width 0.4) (layer F.Cu) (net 3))
 (via (at 142.7117 109.1097) (size 0.4) (layers F.Cu B.Cu) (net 5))
 (segment (start 137.16 107.95) (end 138.4103 107.95) (width 0.4) (layer B.Cu) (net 5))
 (segment (start 143.1925 110.11) (end 143.1925 109.1097) (width 0.4) (layer F.Cu) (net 5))
 (segment (start 142.4488 109.3726) (end 142.7117 109.1097) (width 0.4) (layer B.Cu) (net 5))
 (segment (start 139.8329 109.3726) (end 142.4488 109.3726) (width 0.4) (layer B.Cu) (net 5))
 (segment (start 138.4103 107.95) (end 139.8329 109.3726) (width 0.4) (layer B.Cu) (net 5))
 (segment (start 143.1925 109.1097) (end 142.7117 109.1097) (width 0.4) (layer F.Cu) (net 5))
 (segment (start 137.16 110.49) (end 138.4103 110.49) (width 0.4) (layer F.Cu) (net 6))
 (segment (start 144.4625 110.11) (end 144.4625 111.1103) (width 0.4) (layer F.Cu) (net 6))
 (segment (start 144.4624 111.1103) (end 144.4625 111.1103) (width 0.4) (layer F.Cu) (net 6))
 (segment (start 144.4624 111.3243) (end 144.4624 111.1103) (width 0.4) (layer F.Cu) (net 6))
 (segment (start 144.0761 111.7106) (end 144.4624 111.3243) (width 0.4) (layer F.Cu) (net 6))
 (segment (start 139.6309 111.7106) (end 144.0761 111.7106) (width 0.4) (layer F.Cu) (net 6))
 (segment (start 138.4103 110.49) (end 139.6309 111.7106) (width 0.4) (layer F.Cu) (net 6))
 (segment (start 160.02 100.33) (end 158.7697 100.33) (width 0.4) (layer F.Cu) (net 7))
 (segment (start 145.7325 110.11) (end 145.7325 109.1097) (width 0.4) (layer F.Cu) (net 7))
 (segment (start 149.0485 105.7937) (end 145.7325 109.1097) (width 0.4) (layer F.Cu) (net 7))
 (segment (start 154.3219 105.7937) (end 149.0485 105.7937) (width 0.4) (layer F.Cu) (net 7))
 (segment (start 158.7697 101.3459) (end 154.3219 105.7937) (width 0.4) (layer F.Cu) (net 7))
 (segment (start 158.7697 100.33) (end 158.7697 101.3459) (width 0.4) (layer F.Cu) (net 7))
 (segment (start 154.1631 106.3941) (end 151.4475 109.1097) (width 0.4) (layer F.Cu) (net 8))
 (segment (start 155.2456 106.3941) (end 154.1631 106.3941) (width 0.4) (layer F.Cu) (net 8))
 (segment (start 158.7697 102.87) (end 155.2456 106.3941) (width 0.4) (layer F.Cu) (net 8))
 (segment (start 160.02 102.87) (end 158.7697 102.87) (width 0.4) (layer F.Cu) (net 8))
 (segment (start 151.4475 110.11) (end 151.4475 109.1097) (width 0.4) (layer F.Cu) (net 8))
 (segment (start 152.7175 110.11) (end 152.7175 109.1097) (width 0.4) (layer F.Cu) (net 9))
 (segment (start 160.02 105.41) (end 158.7697 105.41) (width 0.4) (layer F.Cu) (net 9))
 (segment (start 154.614 107.2132) (end 152.7175 109.1097) (width 0.4) (layer F.Cu) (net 9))
 (segment (start 156.9665 107.2132) (end 154.614 107.2132) (width 0.4) (layer F.Cu) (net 9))
 (segment (start 158.7697 105.41) (end 156.9665 107.2132) (width 0.4) (layer F.Cu) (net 9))
 (segment (start 153.9875 110.11) (end 153.9875 109.1097) (width 0.4) (layer F.Cu) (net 10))
 (segment (start 155.1472 107.95) (end 153.9875 109.1097) (width 0.4) (layer F.Cu) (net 10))
 (segment (start 160.02 107.95) (end 155.1472 107.95) (width 0.4) (layer F.Cu) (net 10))
 (segment (start 158.1494 111.1103) (end 155.2575 111.1103) (width 0.4) (layer F.Cu) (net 11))
 (segment (start 158.7697 110.49) (end 158.1494 111.1103) (width 0.4) (layer F.Cu) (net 11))
 (segment (start 160.02 110.49) (end 158.7697 110.49) (width 0.4) (layer F.Cu) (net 11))
 (segment (start 155.2575 110.11) (end 155.2575 111.1103) (width 0.4) (layer F.Cu) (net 11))
 (segment (start 157.1625 99.5719) (end 157.1625 100.71) (width 0.4) (layer F.Cu) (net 14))
 (segment (start 156.2296 98.639) (end 157.1625 99.5719) (width 0.4) (layer F.Cu) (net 14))
 (segment (start 156.2296 97.2037) (end 156.2296 98.639) (width 0.4) (layer F.Cu) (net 14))
 (segment (start 156.933 96.5003) (end 156.2296 97.2037) (width 0.4) (layer F.Cu) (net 14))
 (segment (start 157.48 96.5003) (end 156.933 96.5003) (width 0.4) (layer F.Cu) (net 14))
 (segment (start 157.48 95.25) (end 157.48 96.5003) (width 0.4) (layer F.Cu) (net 14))
 (segment (start 157.546 101.7103) (end 156.5275 101.7103) (width 0.4) (layer F.Cu) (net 15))
 (segment (start 157.8022 101.4541) (end 157.546 101.7103) (width 0.4) (layer F.Cu) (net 15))
 (segment (start 157.8022 99.3625) (end 157.8022 101.4541) (width 0.4) (layer F.Cu) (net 15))
 (segment (start 157.48 99.0403) (end 157.8022 99.3625) (width 0.4) (layer F.Cu) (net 15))
 (segment (start 157.48 97.79) (end 157.48 99.0403) (width 0.4) (layer F.Cu) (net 15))
 (segment (start 156.5275 100.71) (end 156.5275 101.7103) (width 0.4) (layer F.Cu) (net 15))
 (via (at 156.2098 99.7097) (size 0.4) (layers F.Cu B.Cu) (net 16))
 (segment (start 155.8925 100.71) (end 155.8925 99.7097) (width 0.4) (layer F.Cu) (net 16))
 (segment (start 154.94 95.25) (end 154.94 96.5003) (width 0.4) (layer B.Cu) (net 16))
 (segment (start 156.2098 97.2231) (end 156.2098 99.7097) (width 0.4) (layer B.Cu) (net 16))
 (segment (start 155.487 96.5003) (end 156.2098 97.2231) (width 0.4) (layer B.Cu) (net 16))
 (segment (start 154.94 96.5003) (end 155.487 96.5003) (width 0.4) (layer B.Cu) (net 16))
 (segment (start 155.8925 99.7097) (end 156.2098 99.7097) (width 0.4) (layer F.Cu) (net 16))
 (segment (start 154.94 97.79) (end 154.94 99.0403) (width 0.4) (layer F.Cu) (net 17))
 (segment (start 155.2575 99.3578) (end 155.2575 100.71) (width 0.4) (layer F.Cu) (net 17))
 (segment (start 154.94 99.0403) (end 155.2575 99.3578) (width 0.4) (layer F.Cu) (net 17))
 (segment (start 152.9181 96.5003) (end 152.4 96.5003) (width 0.4) (layer F.Cu) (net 18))
 (segment (start 153.67 97.2522) (end 152.9181 96.5003) (width 0.4) (layer F.Cu) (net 18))
 (segment (start 153.67 98.7572) (end 153.67 97.2522) (width 0.4) (layer F.Cu) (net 18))
 (segment (start 154.6225 99.7097) (end 153.67 98.7572) (width 0.4) (layer F.Cu) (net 18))
 (segment (start 154.6225 100.71) (end 154.6225 99.7097) (width 0.4) (layer F.Cu) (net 18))
 (segment (start 152.4 95.25) (end 152.4 96.5003) (width 0.4) (layer F.Cu) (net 18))
 (via (at 153.8964 101.7146) (size 0.4) (layers F.Cu B.Cu) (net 19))
 (segment (start 152.4 100.2182) (end 153.8964 101.7146) (width 0.4) (layer B.Cu) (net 19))
 (segment (start 152.4 97.79) (end 152.4 100.2182) (width 0.4) (layer B.Cu) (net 19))
 (segment (start 153.9007 101.7103) (end 153.8964 101.7146) (width 0.4) (layer F.Cu) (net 19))
 (segment (start 153.9875 101.7103) (end 153.9007 101.7103) (width 0.4) (layer F.Cu) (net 19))
 (segment (start 153.9875 100.71) (end 153.9875 101.7103) (width 0.4) (layer F.Cu) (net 19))
 (via (at 153.4111 99.6923) (size 0.4) (layers F.Cu B.Cu) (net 20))
 (segment (start 153.67 99.4334) (end 153.4111 99.6923) (width 0.4) (layer B.Cu) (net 20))
 (segment (start 153.67 97.2238) (end 153.67 99.4334) (width 0.4) (layer B.Cu) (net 20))
 (segment (start 152.9465 96.5003) (end 153.67 97.2238) (width 0.4) (layer B.Cu) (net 20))
 (segment (start 151.8135 96.5003) (end 152.9465 96.5003) (width 0.4) (layer B.Cu) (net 20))
 (segment (start 151.1103 95.7971) (end 151.8135 96.5003) (width 0.4) (layer B.Cu) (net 20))
 (segment (start 151.1103 95.25) (end 151.1103 95.7971) (width 0.4) (layer B.Cu) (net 20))
 (segment (start 153.3937 99.7097) (end 153.3525 99.7097) (width 0.4) (layer F.Cu) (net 20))
 (segment (start 153.4111 99.6923) (end 153.3937 99.7097) (width 0.4) (layer F.Cu) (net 20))
 (segment (start 153.3525 100.71) (end 153.3525 99.7097) (width 0.4) (layer F.Cu) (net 20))
 (segment (start 149.86 95.25) (end 151.1103 95.25) (width 0.4) (layer B.Cu) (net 20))
 (segment (start 152.5386 99.7097) (end 152.7175 99.7097) (width 0.4) (layer F.Cu) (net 21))
 (segment (start 151.1103 98.2814) (end 152.5386 99.7097) (width 0.4) (layer F.Cu) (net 21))
 (segment (start 151.1103 97.79) (end 151.1103 98.2814) (width 0.4) (layer F.Cu) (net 21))
 (segment (start 149.86 97.79) (end 151.1103 97.79) (width 0.4) (layer F.Cu) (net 21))
 (segment (start 152.7175 100.71) (end 152.7175 99.7097) (width 0.4) (layer F.Cu) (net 21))
 (segment (start 148.5703 98.3081) (end 148.5703 97.79) (width 0.4) (layer F.Cu) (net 23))
 (segment (start 149.3663 99.1041) (end 148.5703 98.3081) (width 0.4) (layer F.Cu) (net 23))
 (segment (start 150.8419 99.1041) (end 149.3663 99.1041) (width 0.4) (layer F.Cu) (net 23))
 (segment (start 151.4475 99.7097) (end 150.8419 99.1041) (width 0.4) (layer F.Cu) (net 23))
 (segment (start 147.32 97.79) (end 148.5703 97.79) (width 0.4) (layer F.Cu) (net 23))
 (segment (start 151.4475 100.71) (end 151.4475 99.7097) (width 0.4) (layer F.Cu) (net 23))
 (segment (start 146.3675 98.6214) (end 146.3675 100.71) (width 0.4) (layer F.Cu) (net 24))
 (segment (start 146.0303 98.2842) (end 146.3675 98.6214) (width 0.4) (layer F.Cu) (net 24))
 (segment (start 146.0303 97.2035) (end 146.0303 98.2842) (width 0.4) (layer F.Cu) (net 24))
 (segment (start 145.3271 96.5003) (end 146.0303 97.2035) (width 0.4) (layer F.Cu) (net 24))
 (segment (start 144.78 96.5003) (end 145.3271 96.5003) (width 0.4) (layer F.Cu) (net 24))
 (segment (start 144.78 95.25) (end 144.78 96.5003) (width 0.4) (layer F.Cu) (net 24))
 (segment (start 144.78 97.79) (end 144.78 99.0403) (width 0.4) (layer F.Cu) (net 25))
 (segment (start 145.7325 100.71) (end 145.7325 99.7097) (width 0.4) (layer F.Cu) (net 25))
 (segment (start 145.2954 99.0403) (end 144.78 99.0403) (width 0.4) (layer F.Cu) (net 25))
 (segment (start 145.7325 99.4774) (end 145.2954 99.0403) (width 0.4) (layer F.Cu) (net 25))
 (segment (start 145.7325 99.7097) (end 145.7325 99.4774) (width 0.4) (layer F.Cu) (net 25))
 (via (at 145.0629 99.7086) (size 0.4) (layers F.Cu B.Cu) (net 26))
 (segment (start 145.0975 99.9238) (end 145.0975 100.71) (width 0.4) (layer F.Cu) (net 26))
 (segment (start 145.0629 99.8892) (end 145.0975 99.9238) (width 0.4) (layer F.Cu) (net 26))
 (segment (start 145.0629 99.7085) (end 145.0629 99.7086) (width 0.4) (layer B.Cu) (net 26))
 (segment (start 144.9015 99.7085) (end 145.0629 99.7085) (width 0.4) (layer B.Cu) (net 26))
 (segment (start 143.4903 98.2973) (end 144.9015 99.7085) (width 0.4) (layer B.Cu) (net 26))
 (segment (start 143.4903 97.2035) (end 143.4903 98.2973) (width 0.4) (layer B.Cu) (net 26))
 (segment (start 142.7871 96.5003) (end 143.4903 97.2035) (width 0.4) (layer B.Cu) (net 26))
 (segment (start 142.24 96.5003) (end 142.7871 96.5003) (width 0.4) (layer B.Cu) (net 26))
 (segment (start 145.0629 99.7086) (end 145.0629 99.8892) (width 0.3998) (layer F.Cu) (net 26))
 (segment (start 142.24 95.25) (end 142.24 96.5003) (width 0.4) (layer B.Cu) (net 26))
 (segment (start 143.4903 98.7375) (end 144.4625 99.7097) (width 0.4) (layer F.Cu) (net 27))
 (segment (start 143.4903 97.79) (end 143.4903 98.7375) (width 0.4) (layer F.Cu) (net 27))
 (segment (start 142.24 97.79) (end 143.4903 97.79) (width 0.4) (layer F.Cu) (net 27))
 (segment (start 144.4625 100.71) (end 144.4625 99.7097) (width 0.4) (layer F.Cu) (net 27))
 (via (at 151.9605 101.7103) (size 0.4) (layers F.Cu B.Cu) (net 22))
 (segment (start 152.0825 100.71) (end 152.0825 101.7103) (width 0.4) (layer F.Cu) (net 22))
 (segment (start 147.32 95.25) (end 147.32 96.5003) (width 0.4) (layer B.Cu) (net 22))
 (segment (start 148.5703 98.3201) (end 151.9605 101.7103) (width 0.4) (layer B.Cu) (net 22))
 (segment (start 148.5703 97.2035) (end 148.5703 98.3201) (width 0.4) (layer B.Cu) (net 22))
 (segment (start 147.8671 96.5003) (end 148.5703 97.2035) (width 0.4) (layer B.Cu) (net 22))
 (segment (start 147.32 96.5003) (end 147.8671 96.5003) (width 0.4) (layer B.Cu) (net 22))
 (segment (start 151.9605 101.7103) (end 152.0825 101.7103) (width 0.4) (layer F.Cu) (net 22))
 (via (at 143.8275 101.7103) (size 0.4) (layers F.Cu B.Cu) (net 28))
 (segment (start 143.8275 100.71) (end 143.8275 101.7103) (width 0.4) (layer F.Cu) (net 28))
 (segment (start 139.7 95.25) (end 139.7 96.5003) (width 0.4) (layer B.Cu) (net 28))
 (segment (start 140.9503 98.8331) (end 143.8275 101.7103) (width 0.4) (layer B.Cu) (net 28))
 (segment (start 140.9503 97.2035) (end 140.9503 98.8331) (width 0.4) (layer B.Cu) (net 28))
 (segment (start 140.2471 96.5003) (end 140.9503 97.2035) (width 0.4) (layer B.Cu) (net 28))
 (segment (start 139.7 96.5003) (end 140.2471 96.5003) (width 0.4) (layer B.Cu) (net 28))
 (segment (start 142.3229 99.7097) (end 143.1925 99.7097) (width 0.4) (layer F.Cu) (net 29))
 (segment (start 140.9503 98.3371) (end 142.3229 99.7097) (width 0.4) (layer F.Cu) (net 29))
 (segment (start 140.9503 97.79) (end 140.9503 98.3371) (width 0.4) (layer F.Cu) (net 29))
 (segment (start 139.7 97.79) (end 140.9503 97.79) (width 0.4) (layer F.Cu) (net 29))
 (segment (start 143.1925 100.71) (end 143.1925 99.7097) (width 0.4) (layer F.Cu) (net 29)))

